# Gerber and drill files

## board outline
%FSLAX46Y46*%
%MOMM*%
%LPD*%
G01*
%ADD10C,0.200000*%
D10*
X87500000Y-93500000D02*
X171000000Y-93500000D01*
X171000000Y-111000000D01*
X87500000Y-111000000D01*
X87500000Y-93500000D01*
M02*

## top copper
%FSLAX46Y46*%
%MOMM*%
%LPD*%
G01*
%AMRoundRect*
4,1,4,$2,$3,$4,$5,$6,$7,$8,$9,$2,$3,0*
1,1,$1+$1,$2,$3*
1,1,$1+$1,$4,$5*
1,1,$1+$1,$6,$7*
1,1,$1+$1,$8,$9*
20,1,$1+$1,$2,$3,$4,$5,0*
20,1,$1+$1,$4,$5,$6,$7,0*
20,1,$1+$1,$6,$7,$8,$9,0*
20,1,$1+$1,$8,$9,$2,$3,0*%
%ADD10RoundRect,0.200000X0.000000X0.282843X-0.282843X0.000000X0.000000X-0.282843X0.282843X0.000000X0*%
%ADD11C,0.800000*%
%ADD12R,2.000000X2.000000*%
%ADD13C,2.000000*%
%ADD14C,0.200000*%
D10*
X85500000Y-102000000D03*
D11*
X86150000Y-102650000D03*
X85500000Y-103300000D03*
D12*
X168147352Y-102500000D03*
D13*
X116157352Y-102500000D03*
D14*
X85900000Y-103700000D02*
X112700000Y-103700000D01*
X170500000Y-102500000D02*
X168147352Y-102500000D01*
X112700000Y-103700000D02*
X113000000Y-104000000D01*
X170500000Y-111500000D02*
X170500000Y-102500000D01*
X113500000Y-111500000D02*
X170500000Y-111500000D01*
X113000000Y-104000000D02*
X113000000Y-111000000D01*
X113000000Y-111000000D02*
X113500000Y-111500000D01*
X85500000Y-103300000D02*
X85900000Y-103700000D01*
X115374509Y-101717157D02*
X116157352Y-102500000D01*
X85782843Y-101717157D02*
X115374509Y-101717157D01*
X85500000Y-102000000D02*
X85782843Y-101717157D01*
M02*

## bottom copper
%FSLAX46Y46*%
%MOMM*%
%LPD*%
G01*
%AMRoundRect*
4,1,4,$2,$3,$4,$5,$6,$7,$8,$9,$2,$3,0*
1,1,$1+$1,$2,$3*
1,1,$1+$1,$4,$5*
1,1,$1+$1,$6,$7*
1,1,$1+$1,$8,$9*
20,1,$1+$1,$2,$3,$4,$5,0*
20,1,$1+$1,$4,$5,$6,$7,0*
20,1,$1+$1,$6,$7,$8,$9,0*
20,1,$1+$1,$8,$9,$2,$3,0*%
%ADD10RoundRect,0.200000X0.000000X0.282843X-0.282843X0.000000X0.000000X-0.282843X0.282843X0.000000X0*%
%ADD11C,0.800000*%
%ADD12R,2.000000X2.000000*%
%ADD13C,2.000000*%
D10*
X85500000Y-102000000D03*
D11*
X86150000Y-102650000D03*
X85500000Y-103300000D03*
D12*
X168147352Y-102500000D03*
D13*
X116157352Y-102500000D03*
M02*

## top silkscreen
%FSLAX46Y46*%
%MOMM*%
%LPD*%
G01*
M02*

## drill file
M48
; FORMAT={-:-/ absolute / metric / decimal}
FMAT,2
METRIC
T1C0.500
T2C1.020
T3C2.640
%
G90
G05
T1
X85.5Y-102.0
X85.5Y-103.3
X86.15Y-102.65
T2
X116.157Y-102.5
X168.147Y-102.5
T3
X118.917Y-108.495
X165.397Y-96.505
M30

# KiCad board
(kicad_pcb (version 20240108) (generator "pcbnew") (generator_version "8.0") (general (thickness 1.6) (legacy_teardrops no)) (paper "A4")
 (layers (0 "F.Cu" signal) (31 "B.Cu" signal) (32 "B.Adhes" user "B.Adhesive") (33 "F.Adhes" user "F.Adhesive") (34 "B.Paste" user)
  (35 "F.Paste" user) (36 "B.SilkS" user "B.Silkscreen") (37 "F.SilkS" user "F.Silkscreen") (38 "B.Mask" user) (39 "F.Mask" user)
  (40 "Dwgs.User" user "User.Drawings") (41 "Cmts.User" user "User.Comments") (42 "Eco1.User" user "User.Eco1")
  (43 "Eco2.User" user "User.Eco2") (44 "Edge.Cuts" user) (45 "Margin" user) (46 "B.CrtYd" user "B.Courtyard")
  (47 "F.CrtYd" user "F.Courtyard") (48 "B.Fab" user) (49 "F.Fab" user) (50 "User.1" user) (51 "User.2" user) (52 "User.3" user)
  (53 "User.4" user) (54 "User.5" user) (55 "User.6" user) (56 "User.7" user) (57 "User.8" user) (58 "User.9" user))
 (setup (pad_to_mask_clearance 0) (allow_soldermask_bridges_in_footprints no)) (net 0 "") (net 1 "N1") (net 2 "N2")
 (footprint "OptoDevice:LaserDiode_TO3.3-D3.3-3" (layer "B.Cu") (at 85.5 102 -90)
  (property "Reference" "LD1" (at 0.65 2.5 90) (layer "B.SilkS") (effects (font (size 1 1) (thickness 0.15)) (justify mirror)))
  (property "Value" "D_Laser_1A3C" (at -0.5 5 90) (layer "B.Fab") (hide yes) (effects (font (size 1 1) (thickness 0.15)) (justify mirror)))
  (pad "1" thru_hole roundrect (at 0 0 225) (size 0.8 0.8) (drill 0.5) (layers "*.Cu" "*.Mask") (remove_unused_layers no)
   (roundrect_rratio 0.25) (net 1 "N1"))
  (pad "2" thru_hole circle (at 0.65 -0.65 270) (size 0.8 0.8) (drill 0.5) (layers "*.Cu" "*.Mask") (remove_unused_layers no))
  (pad "3" thru_hole circle (at 1.3 0 270) (size 0.8 0.8) (drill 0.5) (layers "*.Cu" "*.Mask") (remove_unused_layers no) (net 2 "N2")))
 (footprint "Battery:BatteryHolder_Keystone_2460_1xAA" (layer "B.Cu") (at 168.147352 102.5 180)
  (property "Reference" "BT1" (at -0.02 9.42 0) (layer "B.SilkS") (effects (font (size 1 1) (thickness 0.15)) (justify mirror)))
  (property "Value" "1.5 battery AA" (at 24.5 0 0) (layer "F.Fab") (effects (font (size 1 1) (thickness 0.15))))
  (pad "" np_thru_hole circle (at 2.75 5.995 90) (size 2.64 2.64) (drill 2.64) (layers "*.Cu" "*.Mask"))
  (pad "" np_thru_hole circle (at 49.23 -5.995 180) (size 2.64 2.64) (drill 2.64) (layers "*.Cu" "*.Mask"))
  (pad "1" thru_hole rect (at 0 0) (size 2 2) (drill 1.02) (layers "*.Cu" "*.Mask") (remove_unused_layers no) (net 2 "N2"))
  (pad "2" thru_hole circle (at 51.99 0) (size 2 2) (drill 1.02) (layers "*.Cu" "*.Mask") (remove_unused_layers no) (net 1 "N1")))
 (gr_rect (start 87.5 93.5) (end 171 111) (locked yes) (stroke (width 0.2) (type default)) (fill none) (layer "Edge.Cuts"))
 (segment (start 85.9 103.7) (end 112.7 103.7) (width 0.2) (layer "F.Cu") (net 2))
 (segment (start 170.5 102.5) (end 168.147352 102.5) (width 0.2) (layer "F.Cu") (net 2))
 (segment (start 112.7 103.7) (end 113 104) (width 0.2) (layer "F.Cu") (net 2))
 (segment (start 170.5 111.5) (end 170.5 102.5) (width 0.2) (layer "F.Cu") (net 2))
 (segment (start 113.5 111.5) (end 170.5 111.5) (width 0.2) (layer "F.Cu") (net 2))
 (segment (start 113 104) (end 113 111) (width 0.2) (layer "F.Cu") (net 2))
 (segment (start 113 111) (end 113.5 111.5) (width 0.2) (layer "F.Cu") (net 2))
 (segment (start 85.5 103.3) (end 85.9 103.7) (width 0.2) (layer "F.Cu") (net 2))
 (segment (start 115.374509 101.717157) (end 116.157352 102.5) (width 0.2) (layer "F.Cu") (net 1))
 (segment (start 85.782843 101.717157) (end 115.374509 101.717157) (width 0.2) (layer "F.Cu") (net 1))
 (segment (start 85.5 102) (end 85.782843 101.717157) (width 0.2) (layer "F.Cu") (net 1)))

